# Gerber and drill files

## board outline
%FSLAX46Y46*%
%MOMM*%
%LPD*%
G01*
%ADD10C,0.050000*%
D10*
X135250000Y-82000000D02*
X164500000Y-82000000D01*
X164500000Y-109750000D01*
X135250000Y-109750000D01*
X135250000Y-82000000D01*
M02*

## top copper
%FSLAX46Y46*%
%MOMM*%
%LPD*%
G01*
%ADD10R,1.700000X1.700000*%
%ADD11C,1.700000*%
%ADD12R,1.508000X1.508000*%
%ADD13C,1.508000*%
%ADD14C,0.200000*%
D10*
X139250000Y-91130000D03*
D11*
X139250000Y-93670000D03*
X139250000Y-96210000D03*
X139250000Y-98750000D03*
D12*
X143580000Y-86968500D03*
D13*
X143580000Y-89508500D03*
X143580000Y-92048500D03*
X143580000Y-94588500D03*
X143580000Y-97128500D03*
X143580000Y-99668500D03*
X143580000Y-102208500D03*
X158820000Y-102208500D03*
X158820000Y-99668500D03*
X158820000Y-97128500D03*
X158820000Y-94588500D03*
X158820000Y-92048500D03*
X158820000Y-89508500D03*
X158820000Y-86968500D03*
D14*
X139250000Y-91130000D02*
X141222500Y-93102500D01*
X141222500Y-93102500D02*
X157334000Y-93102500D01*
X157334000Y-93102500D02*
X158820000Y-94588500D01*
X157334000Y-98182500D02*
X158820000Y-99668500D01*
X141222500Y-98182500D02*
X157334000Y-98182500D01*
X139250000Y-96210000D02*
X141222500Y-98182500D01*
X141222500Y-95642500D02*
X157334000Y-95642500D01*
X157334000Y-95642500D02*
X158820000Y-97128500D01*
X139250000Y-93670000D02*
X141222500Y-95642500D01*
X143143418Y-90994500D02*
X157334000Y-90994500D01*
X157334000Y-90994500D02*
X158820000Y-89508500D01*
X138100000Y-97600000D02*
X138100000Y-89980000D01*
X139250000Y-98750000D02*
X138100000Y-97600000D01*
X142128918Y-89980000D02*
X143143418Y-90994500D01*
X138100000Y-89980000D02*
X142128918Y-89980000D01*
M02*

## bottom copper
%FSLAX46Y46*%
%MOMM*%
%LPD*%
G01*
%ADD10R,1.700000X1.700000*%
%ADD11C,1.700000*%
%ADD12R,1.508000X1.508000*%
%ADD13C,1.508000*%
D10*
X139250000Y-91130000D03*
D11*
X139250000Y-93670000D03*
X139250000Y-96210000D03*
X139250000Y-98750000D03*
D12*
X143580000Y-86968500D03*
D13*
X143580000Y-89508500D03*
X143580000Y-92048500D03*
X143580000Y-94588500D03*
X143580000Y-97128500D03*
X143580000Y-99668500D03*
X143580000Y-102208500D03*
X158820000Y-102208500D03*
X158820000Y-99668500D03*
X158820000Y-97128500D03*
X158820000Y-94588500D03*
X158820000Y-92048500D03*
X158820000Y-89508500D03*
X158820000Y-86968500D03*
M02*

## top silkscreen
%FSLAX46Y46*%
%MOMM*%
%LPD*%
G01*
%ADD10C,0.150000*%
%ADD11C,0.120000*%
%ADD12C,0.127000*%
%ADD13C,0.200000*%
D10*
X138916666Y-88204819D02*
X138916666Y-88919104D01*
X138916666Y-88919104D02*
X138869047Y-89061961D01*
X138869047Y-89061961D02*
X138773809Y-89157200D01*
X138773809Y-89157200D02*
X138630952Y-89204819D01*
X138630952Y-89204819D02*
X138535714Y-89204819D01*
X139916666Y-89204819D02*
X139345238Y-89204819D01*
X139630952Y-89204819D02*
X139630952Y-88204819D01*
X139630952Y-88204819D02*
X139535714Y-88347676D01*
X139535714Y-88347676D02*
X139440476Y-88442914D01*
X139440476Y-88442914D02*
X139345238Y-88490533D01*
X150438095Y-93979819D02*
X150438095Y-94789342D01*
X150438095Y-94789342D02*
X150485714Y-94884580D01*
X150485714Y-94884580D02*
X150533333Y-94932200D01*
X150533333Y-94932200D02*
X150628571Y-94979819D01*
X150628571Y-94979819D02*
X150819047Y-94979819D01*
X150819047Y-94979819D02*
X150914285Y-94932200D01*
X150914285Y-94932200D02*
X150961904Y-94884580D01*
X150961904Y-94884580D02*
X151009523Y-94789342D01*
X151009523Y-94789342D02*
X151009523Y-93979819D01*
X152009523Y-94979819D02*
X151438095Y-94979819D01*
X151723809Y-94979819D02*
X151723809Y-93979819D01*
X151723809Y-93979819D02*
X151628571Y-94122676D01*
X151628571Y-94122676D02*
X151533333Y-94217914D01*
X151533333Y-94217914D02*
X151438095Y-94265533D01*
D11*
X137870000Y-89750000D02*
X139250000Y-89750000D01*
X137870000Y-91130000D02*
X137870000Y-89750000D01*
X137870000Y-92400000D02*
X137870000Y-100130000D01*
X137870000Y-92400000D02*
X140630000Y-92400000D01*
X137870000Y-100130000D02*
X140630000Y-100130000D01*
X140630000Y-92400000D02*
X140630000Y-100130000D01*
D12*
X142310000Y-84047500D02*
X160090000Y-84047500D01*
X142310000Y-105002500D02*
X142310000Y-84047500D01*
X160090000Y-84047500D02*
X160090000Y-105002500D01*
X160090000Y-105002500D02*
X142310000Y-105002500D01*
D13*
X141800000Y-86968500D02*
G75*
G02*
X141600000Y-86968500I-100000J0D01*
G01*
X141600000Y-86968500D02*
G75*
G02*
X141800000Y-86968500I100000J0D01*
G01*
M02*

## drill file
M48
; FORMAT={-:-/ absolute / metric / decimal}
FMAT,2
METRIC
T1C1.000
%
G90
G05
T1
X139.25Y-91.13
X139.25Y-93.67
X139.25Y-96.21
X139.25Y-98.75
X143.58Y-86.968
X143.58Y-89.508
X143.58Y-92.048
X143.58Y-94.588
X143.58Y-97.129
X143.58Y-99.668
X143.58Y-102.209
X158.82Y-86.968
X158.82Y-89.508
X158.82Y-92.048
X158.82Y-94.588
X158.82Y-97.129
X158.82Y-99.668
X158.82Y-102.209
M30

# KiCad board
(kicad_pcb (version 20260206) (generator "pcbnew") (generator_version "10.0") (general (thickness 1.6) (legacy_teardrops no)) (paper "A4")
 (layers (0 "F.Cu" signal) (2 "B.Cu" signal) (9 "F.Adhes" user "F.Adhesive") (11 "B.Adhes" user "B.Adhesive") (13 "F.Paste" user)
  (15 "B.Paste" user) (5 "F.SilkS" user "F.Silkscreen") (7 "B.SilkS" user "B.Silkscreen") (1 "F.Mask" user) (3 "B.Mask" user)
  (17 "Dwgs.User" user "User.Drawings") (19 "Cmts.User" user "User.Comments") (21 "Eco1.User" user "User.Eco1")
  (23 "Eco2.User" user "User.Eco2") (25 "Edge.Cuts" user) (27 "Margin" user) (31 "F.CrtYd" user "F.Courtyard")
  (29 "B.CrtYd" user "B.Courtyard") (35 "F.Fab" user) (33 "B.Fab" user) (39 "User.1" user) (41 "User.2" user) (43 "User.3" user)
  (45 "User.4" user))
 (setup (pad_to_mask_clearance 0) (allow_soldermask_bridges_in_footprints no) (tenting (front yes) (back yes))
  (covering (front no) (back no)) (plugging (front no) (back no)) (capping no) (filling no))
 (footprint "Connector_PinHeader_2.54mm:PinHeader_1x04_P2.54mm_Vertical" (layer "F.Cu") (at 139.25 91.13)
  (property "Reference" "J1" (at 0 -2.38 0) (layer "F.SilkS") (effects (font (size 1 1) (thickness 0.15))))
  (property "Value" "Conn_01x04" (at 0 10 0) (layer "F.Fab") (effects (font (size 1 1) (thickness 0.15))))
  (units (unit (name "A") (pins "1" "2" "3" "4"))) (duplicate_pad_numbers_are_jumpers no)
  (fp_line (start -1.38 -1.38) (end 0 -1.38) (stroke (width 0.12) (type solid)) (layer "F.SilkS"))
  (fp_line (start -1.38 0) (end -1.38 -1.38) (stroke (width 0.12) (type solid)) (layer "F.SilkS"))
  (fp_line (start -1.38 1.27) (end -1.38 9) (stroke (width 0.12) (type solid)) (layer "F.SilkS"))
  (fp_line (start -1.38 1.27) (end 1.38 1.27) (stroke (width 0.12) (type solid)) (layer "F.SilkS"))
  (fp_line (start -1.38 9) (end 1.38 9) (stroke (width 0.12) (type solid)) (layer "F.SilkS"))
  (fp_line (start 1.38 1.27) (end 1.38 9) (stroke (width 0.12) (type solid)) (layer "F.SilkS"))
  (pad "1" thru_hole rect (at 0 0) (size 1.7 1.7) (drill 1) (layers "*.Cu" "*.Mask") (remove_unused_layers no) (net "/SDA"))
  (pad "2" thru_hole circle (at 0 2.54) (size 1.7 1.7) (drill 1) (layers "*.Cu" "*.Mask") (remove_unused_layers no) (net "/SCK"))
  (pad "3" thru_hole circle (at 0 5.08) (size 1.7 1.7) (drill 1) (layers "*.Cu" "*.Mask") (remove_unused_layers no) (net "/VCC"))
  (pad "4" thru_hole circle (at 0 7.62) (size 1.7 1.7) (drill 1) (layers "*.Cu" "*.Mask") (remove_unused_layers no) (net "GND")))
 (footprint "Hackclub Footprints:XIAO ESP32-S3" (layer "F.Cu") (at 151.2 94.525)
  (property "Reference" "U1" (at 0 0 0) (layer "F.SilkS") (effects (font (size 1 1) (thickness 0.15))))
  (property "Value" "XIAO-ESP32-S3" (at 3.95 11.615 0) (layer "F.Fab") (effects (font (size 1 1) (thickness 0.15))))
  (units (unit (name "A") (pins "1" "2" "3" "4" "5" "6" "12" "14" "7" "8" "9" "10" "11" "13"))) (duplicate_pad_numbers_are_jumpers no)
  (fp_line (start -8.89 -10.4775) (end 8.89 -10.4775) (stroke (width 0.127) (type solid)) (layer "F.SilkS"))
  (fp_line (start -8.89 10.4775) (end -8.89 -10.4775) (stroke (width 0.127) (type solid)) (layer "F.SilkS"))
  (fp_line (start 8.89 -10.4775) (end 8.89 10.4775) (stroke (width 0.127) (type solid)) (layer "F.SilkS"))
  (fp_line (start 8.89 10.4775) (end -8.89 10.4775) (stroke (width 0.127) (type solid)) (layer "F.SilkS"))
  (fp_circle (center -9.5 -7.5565) (end -9.4 -7.5565) (stroke (width 0.2) (type solid)) (fill no) (layer "F.SilkS"))
  (pad "1" thru_hole rect (at -7.62 -7.5565) (size 1.508 1.508) (drill 1) (layers "*.Cu" "*.Mask") (remove_unused_layers no)
   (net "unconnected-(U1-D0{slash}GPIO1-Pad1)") (solder_mask_margin 0.102))
  (pad "2" thru_hole circle (at -7.62 -5.0165) (size 1.508 1.508) (drill 1) (layers "*.Cu" "*.Mask") (remove_unused_layers no)
   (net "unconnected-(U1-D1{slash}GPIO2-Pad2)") (solder_mask_margin 0.102))
  (pad "3" thru_hole circle (at -7.62 -2.4765) (size 1.508 1.508) (drill 1) (layers "*.Cu" "*.Mask") (remove_unused_layers no)
   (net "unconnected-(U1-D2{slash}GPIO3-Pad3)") (solder_mask_margin 0.102))
  (pad "4" thru_hole circle (at -7.62 0.0635) (size 1.508 1.508) (drill 1) (layers "*.Cu" "*.Mask") (remove_unused_layers no)
   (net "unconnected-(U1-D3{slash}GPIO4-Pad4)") (solder_mask_margin 0.102))
  (pad "5" thru_hole circle (at -7.62 2.6035) (size 1.508 1.508) (drill 1) (layers "*.Cu" "*.Mask") (remove_unused_layers no)
   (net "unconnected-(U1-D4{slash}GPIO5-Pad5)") (solder_mask_margin 0.102))
  (pad "6" thru_hole circle (at -7.62 5.1435) (size 1.508 1.508) (drill 1) (layers "*.Cu" "*.Mask") (remove_unused_layers no)
   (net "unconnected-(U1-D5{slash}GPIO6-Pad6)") (solder_mask_margin 0.102))
  (pad "7" thru_hole circle (at -7.62 7.6835) (size 1.508 1.508) (drill 1) (layers "*.Cu" "*.Mask") (remove_unused_layers no)
   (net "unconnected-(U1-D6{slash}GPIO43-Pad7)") (solder_mask_margin 0.102))
  (pad "8" thru_hole circle (at 7.62 7.6835) (size 1.508 1.508) (drill 1) (layers "*.Cu" "*.Mask") (remove_unused_layers no)
   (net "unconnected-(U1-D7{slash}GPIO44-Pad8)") (solder_mask_margin 0.102))
  (pad "9" thru_hole circle (at 7.62 5.1435) (size 1.508 1.508) (drill 1) (layers "*.Cu" "*.Mask") (remove_unused_layers no) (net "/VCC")
   (solder_mask_margin 0.102))
  (pad "10" thru_hole circle (at 7.62 2.6035) (size 1.508 1.508) (drill 1) (layers "*.Cu" "*.Mask") (remove_unused_layers no) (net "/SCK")
   (solder_mask_margin 0.102))
  (pad "11" thru_hole circle (at 7.62 0.0635) (size 1.508 1.508) (drill 1) (layers "*.Cu" "*.Mask") (remove_unused_layers no) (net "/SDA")
   (solder_mask_margin 0.102))
  (pad "12" thru_hole circle (at 7.62 -2.4765) (size 1.508 1.508) (drill 1) (layers "*.Cu" "*.Mask") (remove_unused_layers no) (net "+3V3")
   (solder_mask_margin 0.102))
  (pad "13" thru_hole circle (at 7.62 -5.0165) (size 1.508 1.508) (drill 1) (layers "*.Cu" "*.Mask") (remove_unused_layers no) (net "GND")
   (solder_mask_margin 0.102))
  (pad "14" thru_hole circle (at 7.62 -7.5565) (size 1.508 1.508) (drill 1) (layers "*.Cu" "*.Mask") (remove_unused_layers no)
   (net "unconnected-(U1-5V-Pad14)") (solder_mask_margin 0.102)))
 (gr_rect (start 135.25 82) (end 164.5 109.75) (stroke (width 0.05) (type default)) (fill no) (layer "Edge.Cuts"))
 (segment (start 139.25 91.13) (end 141.2225 93.1025) (width 0.2) (layer "F.Cu") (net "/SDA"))
 (segment (start 141.2225 93.1025) (end 157.334 93.1025) (width 0.2) (layer "F.Cu") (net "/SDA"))
 (segment (start 157.334 93.1025) (end 158.82 94.5885) (width 0.2) (layer "F.Cu") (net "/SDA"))
 (segment (start 157.334 98.1825) (end 158.82 99.6685) (width 0.2) (layer "F.Cu") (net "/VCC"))
 (segment (start 141.2225 98.1825) (end 157.334 98.1825) (width 0.2) (layer "F.Cu") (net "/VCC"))
 (segment (start 139.25 96.21) (end 141.2225 98.1825) (width 0.2) (layer "F.Cu") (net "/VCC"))
 (segment (start 141.2225 95.6425) (end 157.334 95.6425) (width 0.2) (layer "F.Cu") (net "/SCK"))
 (segment (start 157.334 95.6425) (end 158.82 97.1285) (width 0.2) (layer "F.Cu") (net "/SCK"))
 (segment (start 139.25 93.67) (end 141.2225 95.6425) (width 0.2) (layer "F.Cu") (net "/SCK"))
 (segment (start 143.143418 90.9945) (end 157.334 90.9945) (width 0.2) (layer "F.Cu") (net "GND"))
 (segment (start 157.334 90.9945) (end 158.82 89.5085) (width 0.2) (layer "F.Cu") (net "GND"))
 (segment (start 138.1 97.6) (end 138.1 89.98) (width 0.2) (layer "F.Cu") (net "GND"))
 (segment (start 139.25 98.75) (end 138.1 97.6) (width 0.2) (layer "F.Cu") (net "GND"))
 (segment (start 142.128918 89.98) (end 143.143418 90.9945) (width 0.2) (layer "F.Cu") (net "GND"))
 (segment (start 138.1 89.98) (end 142.128918 89.98) (width 0.2) (layer "F.Cu") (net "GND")))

